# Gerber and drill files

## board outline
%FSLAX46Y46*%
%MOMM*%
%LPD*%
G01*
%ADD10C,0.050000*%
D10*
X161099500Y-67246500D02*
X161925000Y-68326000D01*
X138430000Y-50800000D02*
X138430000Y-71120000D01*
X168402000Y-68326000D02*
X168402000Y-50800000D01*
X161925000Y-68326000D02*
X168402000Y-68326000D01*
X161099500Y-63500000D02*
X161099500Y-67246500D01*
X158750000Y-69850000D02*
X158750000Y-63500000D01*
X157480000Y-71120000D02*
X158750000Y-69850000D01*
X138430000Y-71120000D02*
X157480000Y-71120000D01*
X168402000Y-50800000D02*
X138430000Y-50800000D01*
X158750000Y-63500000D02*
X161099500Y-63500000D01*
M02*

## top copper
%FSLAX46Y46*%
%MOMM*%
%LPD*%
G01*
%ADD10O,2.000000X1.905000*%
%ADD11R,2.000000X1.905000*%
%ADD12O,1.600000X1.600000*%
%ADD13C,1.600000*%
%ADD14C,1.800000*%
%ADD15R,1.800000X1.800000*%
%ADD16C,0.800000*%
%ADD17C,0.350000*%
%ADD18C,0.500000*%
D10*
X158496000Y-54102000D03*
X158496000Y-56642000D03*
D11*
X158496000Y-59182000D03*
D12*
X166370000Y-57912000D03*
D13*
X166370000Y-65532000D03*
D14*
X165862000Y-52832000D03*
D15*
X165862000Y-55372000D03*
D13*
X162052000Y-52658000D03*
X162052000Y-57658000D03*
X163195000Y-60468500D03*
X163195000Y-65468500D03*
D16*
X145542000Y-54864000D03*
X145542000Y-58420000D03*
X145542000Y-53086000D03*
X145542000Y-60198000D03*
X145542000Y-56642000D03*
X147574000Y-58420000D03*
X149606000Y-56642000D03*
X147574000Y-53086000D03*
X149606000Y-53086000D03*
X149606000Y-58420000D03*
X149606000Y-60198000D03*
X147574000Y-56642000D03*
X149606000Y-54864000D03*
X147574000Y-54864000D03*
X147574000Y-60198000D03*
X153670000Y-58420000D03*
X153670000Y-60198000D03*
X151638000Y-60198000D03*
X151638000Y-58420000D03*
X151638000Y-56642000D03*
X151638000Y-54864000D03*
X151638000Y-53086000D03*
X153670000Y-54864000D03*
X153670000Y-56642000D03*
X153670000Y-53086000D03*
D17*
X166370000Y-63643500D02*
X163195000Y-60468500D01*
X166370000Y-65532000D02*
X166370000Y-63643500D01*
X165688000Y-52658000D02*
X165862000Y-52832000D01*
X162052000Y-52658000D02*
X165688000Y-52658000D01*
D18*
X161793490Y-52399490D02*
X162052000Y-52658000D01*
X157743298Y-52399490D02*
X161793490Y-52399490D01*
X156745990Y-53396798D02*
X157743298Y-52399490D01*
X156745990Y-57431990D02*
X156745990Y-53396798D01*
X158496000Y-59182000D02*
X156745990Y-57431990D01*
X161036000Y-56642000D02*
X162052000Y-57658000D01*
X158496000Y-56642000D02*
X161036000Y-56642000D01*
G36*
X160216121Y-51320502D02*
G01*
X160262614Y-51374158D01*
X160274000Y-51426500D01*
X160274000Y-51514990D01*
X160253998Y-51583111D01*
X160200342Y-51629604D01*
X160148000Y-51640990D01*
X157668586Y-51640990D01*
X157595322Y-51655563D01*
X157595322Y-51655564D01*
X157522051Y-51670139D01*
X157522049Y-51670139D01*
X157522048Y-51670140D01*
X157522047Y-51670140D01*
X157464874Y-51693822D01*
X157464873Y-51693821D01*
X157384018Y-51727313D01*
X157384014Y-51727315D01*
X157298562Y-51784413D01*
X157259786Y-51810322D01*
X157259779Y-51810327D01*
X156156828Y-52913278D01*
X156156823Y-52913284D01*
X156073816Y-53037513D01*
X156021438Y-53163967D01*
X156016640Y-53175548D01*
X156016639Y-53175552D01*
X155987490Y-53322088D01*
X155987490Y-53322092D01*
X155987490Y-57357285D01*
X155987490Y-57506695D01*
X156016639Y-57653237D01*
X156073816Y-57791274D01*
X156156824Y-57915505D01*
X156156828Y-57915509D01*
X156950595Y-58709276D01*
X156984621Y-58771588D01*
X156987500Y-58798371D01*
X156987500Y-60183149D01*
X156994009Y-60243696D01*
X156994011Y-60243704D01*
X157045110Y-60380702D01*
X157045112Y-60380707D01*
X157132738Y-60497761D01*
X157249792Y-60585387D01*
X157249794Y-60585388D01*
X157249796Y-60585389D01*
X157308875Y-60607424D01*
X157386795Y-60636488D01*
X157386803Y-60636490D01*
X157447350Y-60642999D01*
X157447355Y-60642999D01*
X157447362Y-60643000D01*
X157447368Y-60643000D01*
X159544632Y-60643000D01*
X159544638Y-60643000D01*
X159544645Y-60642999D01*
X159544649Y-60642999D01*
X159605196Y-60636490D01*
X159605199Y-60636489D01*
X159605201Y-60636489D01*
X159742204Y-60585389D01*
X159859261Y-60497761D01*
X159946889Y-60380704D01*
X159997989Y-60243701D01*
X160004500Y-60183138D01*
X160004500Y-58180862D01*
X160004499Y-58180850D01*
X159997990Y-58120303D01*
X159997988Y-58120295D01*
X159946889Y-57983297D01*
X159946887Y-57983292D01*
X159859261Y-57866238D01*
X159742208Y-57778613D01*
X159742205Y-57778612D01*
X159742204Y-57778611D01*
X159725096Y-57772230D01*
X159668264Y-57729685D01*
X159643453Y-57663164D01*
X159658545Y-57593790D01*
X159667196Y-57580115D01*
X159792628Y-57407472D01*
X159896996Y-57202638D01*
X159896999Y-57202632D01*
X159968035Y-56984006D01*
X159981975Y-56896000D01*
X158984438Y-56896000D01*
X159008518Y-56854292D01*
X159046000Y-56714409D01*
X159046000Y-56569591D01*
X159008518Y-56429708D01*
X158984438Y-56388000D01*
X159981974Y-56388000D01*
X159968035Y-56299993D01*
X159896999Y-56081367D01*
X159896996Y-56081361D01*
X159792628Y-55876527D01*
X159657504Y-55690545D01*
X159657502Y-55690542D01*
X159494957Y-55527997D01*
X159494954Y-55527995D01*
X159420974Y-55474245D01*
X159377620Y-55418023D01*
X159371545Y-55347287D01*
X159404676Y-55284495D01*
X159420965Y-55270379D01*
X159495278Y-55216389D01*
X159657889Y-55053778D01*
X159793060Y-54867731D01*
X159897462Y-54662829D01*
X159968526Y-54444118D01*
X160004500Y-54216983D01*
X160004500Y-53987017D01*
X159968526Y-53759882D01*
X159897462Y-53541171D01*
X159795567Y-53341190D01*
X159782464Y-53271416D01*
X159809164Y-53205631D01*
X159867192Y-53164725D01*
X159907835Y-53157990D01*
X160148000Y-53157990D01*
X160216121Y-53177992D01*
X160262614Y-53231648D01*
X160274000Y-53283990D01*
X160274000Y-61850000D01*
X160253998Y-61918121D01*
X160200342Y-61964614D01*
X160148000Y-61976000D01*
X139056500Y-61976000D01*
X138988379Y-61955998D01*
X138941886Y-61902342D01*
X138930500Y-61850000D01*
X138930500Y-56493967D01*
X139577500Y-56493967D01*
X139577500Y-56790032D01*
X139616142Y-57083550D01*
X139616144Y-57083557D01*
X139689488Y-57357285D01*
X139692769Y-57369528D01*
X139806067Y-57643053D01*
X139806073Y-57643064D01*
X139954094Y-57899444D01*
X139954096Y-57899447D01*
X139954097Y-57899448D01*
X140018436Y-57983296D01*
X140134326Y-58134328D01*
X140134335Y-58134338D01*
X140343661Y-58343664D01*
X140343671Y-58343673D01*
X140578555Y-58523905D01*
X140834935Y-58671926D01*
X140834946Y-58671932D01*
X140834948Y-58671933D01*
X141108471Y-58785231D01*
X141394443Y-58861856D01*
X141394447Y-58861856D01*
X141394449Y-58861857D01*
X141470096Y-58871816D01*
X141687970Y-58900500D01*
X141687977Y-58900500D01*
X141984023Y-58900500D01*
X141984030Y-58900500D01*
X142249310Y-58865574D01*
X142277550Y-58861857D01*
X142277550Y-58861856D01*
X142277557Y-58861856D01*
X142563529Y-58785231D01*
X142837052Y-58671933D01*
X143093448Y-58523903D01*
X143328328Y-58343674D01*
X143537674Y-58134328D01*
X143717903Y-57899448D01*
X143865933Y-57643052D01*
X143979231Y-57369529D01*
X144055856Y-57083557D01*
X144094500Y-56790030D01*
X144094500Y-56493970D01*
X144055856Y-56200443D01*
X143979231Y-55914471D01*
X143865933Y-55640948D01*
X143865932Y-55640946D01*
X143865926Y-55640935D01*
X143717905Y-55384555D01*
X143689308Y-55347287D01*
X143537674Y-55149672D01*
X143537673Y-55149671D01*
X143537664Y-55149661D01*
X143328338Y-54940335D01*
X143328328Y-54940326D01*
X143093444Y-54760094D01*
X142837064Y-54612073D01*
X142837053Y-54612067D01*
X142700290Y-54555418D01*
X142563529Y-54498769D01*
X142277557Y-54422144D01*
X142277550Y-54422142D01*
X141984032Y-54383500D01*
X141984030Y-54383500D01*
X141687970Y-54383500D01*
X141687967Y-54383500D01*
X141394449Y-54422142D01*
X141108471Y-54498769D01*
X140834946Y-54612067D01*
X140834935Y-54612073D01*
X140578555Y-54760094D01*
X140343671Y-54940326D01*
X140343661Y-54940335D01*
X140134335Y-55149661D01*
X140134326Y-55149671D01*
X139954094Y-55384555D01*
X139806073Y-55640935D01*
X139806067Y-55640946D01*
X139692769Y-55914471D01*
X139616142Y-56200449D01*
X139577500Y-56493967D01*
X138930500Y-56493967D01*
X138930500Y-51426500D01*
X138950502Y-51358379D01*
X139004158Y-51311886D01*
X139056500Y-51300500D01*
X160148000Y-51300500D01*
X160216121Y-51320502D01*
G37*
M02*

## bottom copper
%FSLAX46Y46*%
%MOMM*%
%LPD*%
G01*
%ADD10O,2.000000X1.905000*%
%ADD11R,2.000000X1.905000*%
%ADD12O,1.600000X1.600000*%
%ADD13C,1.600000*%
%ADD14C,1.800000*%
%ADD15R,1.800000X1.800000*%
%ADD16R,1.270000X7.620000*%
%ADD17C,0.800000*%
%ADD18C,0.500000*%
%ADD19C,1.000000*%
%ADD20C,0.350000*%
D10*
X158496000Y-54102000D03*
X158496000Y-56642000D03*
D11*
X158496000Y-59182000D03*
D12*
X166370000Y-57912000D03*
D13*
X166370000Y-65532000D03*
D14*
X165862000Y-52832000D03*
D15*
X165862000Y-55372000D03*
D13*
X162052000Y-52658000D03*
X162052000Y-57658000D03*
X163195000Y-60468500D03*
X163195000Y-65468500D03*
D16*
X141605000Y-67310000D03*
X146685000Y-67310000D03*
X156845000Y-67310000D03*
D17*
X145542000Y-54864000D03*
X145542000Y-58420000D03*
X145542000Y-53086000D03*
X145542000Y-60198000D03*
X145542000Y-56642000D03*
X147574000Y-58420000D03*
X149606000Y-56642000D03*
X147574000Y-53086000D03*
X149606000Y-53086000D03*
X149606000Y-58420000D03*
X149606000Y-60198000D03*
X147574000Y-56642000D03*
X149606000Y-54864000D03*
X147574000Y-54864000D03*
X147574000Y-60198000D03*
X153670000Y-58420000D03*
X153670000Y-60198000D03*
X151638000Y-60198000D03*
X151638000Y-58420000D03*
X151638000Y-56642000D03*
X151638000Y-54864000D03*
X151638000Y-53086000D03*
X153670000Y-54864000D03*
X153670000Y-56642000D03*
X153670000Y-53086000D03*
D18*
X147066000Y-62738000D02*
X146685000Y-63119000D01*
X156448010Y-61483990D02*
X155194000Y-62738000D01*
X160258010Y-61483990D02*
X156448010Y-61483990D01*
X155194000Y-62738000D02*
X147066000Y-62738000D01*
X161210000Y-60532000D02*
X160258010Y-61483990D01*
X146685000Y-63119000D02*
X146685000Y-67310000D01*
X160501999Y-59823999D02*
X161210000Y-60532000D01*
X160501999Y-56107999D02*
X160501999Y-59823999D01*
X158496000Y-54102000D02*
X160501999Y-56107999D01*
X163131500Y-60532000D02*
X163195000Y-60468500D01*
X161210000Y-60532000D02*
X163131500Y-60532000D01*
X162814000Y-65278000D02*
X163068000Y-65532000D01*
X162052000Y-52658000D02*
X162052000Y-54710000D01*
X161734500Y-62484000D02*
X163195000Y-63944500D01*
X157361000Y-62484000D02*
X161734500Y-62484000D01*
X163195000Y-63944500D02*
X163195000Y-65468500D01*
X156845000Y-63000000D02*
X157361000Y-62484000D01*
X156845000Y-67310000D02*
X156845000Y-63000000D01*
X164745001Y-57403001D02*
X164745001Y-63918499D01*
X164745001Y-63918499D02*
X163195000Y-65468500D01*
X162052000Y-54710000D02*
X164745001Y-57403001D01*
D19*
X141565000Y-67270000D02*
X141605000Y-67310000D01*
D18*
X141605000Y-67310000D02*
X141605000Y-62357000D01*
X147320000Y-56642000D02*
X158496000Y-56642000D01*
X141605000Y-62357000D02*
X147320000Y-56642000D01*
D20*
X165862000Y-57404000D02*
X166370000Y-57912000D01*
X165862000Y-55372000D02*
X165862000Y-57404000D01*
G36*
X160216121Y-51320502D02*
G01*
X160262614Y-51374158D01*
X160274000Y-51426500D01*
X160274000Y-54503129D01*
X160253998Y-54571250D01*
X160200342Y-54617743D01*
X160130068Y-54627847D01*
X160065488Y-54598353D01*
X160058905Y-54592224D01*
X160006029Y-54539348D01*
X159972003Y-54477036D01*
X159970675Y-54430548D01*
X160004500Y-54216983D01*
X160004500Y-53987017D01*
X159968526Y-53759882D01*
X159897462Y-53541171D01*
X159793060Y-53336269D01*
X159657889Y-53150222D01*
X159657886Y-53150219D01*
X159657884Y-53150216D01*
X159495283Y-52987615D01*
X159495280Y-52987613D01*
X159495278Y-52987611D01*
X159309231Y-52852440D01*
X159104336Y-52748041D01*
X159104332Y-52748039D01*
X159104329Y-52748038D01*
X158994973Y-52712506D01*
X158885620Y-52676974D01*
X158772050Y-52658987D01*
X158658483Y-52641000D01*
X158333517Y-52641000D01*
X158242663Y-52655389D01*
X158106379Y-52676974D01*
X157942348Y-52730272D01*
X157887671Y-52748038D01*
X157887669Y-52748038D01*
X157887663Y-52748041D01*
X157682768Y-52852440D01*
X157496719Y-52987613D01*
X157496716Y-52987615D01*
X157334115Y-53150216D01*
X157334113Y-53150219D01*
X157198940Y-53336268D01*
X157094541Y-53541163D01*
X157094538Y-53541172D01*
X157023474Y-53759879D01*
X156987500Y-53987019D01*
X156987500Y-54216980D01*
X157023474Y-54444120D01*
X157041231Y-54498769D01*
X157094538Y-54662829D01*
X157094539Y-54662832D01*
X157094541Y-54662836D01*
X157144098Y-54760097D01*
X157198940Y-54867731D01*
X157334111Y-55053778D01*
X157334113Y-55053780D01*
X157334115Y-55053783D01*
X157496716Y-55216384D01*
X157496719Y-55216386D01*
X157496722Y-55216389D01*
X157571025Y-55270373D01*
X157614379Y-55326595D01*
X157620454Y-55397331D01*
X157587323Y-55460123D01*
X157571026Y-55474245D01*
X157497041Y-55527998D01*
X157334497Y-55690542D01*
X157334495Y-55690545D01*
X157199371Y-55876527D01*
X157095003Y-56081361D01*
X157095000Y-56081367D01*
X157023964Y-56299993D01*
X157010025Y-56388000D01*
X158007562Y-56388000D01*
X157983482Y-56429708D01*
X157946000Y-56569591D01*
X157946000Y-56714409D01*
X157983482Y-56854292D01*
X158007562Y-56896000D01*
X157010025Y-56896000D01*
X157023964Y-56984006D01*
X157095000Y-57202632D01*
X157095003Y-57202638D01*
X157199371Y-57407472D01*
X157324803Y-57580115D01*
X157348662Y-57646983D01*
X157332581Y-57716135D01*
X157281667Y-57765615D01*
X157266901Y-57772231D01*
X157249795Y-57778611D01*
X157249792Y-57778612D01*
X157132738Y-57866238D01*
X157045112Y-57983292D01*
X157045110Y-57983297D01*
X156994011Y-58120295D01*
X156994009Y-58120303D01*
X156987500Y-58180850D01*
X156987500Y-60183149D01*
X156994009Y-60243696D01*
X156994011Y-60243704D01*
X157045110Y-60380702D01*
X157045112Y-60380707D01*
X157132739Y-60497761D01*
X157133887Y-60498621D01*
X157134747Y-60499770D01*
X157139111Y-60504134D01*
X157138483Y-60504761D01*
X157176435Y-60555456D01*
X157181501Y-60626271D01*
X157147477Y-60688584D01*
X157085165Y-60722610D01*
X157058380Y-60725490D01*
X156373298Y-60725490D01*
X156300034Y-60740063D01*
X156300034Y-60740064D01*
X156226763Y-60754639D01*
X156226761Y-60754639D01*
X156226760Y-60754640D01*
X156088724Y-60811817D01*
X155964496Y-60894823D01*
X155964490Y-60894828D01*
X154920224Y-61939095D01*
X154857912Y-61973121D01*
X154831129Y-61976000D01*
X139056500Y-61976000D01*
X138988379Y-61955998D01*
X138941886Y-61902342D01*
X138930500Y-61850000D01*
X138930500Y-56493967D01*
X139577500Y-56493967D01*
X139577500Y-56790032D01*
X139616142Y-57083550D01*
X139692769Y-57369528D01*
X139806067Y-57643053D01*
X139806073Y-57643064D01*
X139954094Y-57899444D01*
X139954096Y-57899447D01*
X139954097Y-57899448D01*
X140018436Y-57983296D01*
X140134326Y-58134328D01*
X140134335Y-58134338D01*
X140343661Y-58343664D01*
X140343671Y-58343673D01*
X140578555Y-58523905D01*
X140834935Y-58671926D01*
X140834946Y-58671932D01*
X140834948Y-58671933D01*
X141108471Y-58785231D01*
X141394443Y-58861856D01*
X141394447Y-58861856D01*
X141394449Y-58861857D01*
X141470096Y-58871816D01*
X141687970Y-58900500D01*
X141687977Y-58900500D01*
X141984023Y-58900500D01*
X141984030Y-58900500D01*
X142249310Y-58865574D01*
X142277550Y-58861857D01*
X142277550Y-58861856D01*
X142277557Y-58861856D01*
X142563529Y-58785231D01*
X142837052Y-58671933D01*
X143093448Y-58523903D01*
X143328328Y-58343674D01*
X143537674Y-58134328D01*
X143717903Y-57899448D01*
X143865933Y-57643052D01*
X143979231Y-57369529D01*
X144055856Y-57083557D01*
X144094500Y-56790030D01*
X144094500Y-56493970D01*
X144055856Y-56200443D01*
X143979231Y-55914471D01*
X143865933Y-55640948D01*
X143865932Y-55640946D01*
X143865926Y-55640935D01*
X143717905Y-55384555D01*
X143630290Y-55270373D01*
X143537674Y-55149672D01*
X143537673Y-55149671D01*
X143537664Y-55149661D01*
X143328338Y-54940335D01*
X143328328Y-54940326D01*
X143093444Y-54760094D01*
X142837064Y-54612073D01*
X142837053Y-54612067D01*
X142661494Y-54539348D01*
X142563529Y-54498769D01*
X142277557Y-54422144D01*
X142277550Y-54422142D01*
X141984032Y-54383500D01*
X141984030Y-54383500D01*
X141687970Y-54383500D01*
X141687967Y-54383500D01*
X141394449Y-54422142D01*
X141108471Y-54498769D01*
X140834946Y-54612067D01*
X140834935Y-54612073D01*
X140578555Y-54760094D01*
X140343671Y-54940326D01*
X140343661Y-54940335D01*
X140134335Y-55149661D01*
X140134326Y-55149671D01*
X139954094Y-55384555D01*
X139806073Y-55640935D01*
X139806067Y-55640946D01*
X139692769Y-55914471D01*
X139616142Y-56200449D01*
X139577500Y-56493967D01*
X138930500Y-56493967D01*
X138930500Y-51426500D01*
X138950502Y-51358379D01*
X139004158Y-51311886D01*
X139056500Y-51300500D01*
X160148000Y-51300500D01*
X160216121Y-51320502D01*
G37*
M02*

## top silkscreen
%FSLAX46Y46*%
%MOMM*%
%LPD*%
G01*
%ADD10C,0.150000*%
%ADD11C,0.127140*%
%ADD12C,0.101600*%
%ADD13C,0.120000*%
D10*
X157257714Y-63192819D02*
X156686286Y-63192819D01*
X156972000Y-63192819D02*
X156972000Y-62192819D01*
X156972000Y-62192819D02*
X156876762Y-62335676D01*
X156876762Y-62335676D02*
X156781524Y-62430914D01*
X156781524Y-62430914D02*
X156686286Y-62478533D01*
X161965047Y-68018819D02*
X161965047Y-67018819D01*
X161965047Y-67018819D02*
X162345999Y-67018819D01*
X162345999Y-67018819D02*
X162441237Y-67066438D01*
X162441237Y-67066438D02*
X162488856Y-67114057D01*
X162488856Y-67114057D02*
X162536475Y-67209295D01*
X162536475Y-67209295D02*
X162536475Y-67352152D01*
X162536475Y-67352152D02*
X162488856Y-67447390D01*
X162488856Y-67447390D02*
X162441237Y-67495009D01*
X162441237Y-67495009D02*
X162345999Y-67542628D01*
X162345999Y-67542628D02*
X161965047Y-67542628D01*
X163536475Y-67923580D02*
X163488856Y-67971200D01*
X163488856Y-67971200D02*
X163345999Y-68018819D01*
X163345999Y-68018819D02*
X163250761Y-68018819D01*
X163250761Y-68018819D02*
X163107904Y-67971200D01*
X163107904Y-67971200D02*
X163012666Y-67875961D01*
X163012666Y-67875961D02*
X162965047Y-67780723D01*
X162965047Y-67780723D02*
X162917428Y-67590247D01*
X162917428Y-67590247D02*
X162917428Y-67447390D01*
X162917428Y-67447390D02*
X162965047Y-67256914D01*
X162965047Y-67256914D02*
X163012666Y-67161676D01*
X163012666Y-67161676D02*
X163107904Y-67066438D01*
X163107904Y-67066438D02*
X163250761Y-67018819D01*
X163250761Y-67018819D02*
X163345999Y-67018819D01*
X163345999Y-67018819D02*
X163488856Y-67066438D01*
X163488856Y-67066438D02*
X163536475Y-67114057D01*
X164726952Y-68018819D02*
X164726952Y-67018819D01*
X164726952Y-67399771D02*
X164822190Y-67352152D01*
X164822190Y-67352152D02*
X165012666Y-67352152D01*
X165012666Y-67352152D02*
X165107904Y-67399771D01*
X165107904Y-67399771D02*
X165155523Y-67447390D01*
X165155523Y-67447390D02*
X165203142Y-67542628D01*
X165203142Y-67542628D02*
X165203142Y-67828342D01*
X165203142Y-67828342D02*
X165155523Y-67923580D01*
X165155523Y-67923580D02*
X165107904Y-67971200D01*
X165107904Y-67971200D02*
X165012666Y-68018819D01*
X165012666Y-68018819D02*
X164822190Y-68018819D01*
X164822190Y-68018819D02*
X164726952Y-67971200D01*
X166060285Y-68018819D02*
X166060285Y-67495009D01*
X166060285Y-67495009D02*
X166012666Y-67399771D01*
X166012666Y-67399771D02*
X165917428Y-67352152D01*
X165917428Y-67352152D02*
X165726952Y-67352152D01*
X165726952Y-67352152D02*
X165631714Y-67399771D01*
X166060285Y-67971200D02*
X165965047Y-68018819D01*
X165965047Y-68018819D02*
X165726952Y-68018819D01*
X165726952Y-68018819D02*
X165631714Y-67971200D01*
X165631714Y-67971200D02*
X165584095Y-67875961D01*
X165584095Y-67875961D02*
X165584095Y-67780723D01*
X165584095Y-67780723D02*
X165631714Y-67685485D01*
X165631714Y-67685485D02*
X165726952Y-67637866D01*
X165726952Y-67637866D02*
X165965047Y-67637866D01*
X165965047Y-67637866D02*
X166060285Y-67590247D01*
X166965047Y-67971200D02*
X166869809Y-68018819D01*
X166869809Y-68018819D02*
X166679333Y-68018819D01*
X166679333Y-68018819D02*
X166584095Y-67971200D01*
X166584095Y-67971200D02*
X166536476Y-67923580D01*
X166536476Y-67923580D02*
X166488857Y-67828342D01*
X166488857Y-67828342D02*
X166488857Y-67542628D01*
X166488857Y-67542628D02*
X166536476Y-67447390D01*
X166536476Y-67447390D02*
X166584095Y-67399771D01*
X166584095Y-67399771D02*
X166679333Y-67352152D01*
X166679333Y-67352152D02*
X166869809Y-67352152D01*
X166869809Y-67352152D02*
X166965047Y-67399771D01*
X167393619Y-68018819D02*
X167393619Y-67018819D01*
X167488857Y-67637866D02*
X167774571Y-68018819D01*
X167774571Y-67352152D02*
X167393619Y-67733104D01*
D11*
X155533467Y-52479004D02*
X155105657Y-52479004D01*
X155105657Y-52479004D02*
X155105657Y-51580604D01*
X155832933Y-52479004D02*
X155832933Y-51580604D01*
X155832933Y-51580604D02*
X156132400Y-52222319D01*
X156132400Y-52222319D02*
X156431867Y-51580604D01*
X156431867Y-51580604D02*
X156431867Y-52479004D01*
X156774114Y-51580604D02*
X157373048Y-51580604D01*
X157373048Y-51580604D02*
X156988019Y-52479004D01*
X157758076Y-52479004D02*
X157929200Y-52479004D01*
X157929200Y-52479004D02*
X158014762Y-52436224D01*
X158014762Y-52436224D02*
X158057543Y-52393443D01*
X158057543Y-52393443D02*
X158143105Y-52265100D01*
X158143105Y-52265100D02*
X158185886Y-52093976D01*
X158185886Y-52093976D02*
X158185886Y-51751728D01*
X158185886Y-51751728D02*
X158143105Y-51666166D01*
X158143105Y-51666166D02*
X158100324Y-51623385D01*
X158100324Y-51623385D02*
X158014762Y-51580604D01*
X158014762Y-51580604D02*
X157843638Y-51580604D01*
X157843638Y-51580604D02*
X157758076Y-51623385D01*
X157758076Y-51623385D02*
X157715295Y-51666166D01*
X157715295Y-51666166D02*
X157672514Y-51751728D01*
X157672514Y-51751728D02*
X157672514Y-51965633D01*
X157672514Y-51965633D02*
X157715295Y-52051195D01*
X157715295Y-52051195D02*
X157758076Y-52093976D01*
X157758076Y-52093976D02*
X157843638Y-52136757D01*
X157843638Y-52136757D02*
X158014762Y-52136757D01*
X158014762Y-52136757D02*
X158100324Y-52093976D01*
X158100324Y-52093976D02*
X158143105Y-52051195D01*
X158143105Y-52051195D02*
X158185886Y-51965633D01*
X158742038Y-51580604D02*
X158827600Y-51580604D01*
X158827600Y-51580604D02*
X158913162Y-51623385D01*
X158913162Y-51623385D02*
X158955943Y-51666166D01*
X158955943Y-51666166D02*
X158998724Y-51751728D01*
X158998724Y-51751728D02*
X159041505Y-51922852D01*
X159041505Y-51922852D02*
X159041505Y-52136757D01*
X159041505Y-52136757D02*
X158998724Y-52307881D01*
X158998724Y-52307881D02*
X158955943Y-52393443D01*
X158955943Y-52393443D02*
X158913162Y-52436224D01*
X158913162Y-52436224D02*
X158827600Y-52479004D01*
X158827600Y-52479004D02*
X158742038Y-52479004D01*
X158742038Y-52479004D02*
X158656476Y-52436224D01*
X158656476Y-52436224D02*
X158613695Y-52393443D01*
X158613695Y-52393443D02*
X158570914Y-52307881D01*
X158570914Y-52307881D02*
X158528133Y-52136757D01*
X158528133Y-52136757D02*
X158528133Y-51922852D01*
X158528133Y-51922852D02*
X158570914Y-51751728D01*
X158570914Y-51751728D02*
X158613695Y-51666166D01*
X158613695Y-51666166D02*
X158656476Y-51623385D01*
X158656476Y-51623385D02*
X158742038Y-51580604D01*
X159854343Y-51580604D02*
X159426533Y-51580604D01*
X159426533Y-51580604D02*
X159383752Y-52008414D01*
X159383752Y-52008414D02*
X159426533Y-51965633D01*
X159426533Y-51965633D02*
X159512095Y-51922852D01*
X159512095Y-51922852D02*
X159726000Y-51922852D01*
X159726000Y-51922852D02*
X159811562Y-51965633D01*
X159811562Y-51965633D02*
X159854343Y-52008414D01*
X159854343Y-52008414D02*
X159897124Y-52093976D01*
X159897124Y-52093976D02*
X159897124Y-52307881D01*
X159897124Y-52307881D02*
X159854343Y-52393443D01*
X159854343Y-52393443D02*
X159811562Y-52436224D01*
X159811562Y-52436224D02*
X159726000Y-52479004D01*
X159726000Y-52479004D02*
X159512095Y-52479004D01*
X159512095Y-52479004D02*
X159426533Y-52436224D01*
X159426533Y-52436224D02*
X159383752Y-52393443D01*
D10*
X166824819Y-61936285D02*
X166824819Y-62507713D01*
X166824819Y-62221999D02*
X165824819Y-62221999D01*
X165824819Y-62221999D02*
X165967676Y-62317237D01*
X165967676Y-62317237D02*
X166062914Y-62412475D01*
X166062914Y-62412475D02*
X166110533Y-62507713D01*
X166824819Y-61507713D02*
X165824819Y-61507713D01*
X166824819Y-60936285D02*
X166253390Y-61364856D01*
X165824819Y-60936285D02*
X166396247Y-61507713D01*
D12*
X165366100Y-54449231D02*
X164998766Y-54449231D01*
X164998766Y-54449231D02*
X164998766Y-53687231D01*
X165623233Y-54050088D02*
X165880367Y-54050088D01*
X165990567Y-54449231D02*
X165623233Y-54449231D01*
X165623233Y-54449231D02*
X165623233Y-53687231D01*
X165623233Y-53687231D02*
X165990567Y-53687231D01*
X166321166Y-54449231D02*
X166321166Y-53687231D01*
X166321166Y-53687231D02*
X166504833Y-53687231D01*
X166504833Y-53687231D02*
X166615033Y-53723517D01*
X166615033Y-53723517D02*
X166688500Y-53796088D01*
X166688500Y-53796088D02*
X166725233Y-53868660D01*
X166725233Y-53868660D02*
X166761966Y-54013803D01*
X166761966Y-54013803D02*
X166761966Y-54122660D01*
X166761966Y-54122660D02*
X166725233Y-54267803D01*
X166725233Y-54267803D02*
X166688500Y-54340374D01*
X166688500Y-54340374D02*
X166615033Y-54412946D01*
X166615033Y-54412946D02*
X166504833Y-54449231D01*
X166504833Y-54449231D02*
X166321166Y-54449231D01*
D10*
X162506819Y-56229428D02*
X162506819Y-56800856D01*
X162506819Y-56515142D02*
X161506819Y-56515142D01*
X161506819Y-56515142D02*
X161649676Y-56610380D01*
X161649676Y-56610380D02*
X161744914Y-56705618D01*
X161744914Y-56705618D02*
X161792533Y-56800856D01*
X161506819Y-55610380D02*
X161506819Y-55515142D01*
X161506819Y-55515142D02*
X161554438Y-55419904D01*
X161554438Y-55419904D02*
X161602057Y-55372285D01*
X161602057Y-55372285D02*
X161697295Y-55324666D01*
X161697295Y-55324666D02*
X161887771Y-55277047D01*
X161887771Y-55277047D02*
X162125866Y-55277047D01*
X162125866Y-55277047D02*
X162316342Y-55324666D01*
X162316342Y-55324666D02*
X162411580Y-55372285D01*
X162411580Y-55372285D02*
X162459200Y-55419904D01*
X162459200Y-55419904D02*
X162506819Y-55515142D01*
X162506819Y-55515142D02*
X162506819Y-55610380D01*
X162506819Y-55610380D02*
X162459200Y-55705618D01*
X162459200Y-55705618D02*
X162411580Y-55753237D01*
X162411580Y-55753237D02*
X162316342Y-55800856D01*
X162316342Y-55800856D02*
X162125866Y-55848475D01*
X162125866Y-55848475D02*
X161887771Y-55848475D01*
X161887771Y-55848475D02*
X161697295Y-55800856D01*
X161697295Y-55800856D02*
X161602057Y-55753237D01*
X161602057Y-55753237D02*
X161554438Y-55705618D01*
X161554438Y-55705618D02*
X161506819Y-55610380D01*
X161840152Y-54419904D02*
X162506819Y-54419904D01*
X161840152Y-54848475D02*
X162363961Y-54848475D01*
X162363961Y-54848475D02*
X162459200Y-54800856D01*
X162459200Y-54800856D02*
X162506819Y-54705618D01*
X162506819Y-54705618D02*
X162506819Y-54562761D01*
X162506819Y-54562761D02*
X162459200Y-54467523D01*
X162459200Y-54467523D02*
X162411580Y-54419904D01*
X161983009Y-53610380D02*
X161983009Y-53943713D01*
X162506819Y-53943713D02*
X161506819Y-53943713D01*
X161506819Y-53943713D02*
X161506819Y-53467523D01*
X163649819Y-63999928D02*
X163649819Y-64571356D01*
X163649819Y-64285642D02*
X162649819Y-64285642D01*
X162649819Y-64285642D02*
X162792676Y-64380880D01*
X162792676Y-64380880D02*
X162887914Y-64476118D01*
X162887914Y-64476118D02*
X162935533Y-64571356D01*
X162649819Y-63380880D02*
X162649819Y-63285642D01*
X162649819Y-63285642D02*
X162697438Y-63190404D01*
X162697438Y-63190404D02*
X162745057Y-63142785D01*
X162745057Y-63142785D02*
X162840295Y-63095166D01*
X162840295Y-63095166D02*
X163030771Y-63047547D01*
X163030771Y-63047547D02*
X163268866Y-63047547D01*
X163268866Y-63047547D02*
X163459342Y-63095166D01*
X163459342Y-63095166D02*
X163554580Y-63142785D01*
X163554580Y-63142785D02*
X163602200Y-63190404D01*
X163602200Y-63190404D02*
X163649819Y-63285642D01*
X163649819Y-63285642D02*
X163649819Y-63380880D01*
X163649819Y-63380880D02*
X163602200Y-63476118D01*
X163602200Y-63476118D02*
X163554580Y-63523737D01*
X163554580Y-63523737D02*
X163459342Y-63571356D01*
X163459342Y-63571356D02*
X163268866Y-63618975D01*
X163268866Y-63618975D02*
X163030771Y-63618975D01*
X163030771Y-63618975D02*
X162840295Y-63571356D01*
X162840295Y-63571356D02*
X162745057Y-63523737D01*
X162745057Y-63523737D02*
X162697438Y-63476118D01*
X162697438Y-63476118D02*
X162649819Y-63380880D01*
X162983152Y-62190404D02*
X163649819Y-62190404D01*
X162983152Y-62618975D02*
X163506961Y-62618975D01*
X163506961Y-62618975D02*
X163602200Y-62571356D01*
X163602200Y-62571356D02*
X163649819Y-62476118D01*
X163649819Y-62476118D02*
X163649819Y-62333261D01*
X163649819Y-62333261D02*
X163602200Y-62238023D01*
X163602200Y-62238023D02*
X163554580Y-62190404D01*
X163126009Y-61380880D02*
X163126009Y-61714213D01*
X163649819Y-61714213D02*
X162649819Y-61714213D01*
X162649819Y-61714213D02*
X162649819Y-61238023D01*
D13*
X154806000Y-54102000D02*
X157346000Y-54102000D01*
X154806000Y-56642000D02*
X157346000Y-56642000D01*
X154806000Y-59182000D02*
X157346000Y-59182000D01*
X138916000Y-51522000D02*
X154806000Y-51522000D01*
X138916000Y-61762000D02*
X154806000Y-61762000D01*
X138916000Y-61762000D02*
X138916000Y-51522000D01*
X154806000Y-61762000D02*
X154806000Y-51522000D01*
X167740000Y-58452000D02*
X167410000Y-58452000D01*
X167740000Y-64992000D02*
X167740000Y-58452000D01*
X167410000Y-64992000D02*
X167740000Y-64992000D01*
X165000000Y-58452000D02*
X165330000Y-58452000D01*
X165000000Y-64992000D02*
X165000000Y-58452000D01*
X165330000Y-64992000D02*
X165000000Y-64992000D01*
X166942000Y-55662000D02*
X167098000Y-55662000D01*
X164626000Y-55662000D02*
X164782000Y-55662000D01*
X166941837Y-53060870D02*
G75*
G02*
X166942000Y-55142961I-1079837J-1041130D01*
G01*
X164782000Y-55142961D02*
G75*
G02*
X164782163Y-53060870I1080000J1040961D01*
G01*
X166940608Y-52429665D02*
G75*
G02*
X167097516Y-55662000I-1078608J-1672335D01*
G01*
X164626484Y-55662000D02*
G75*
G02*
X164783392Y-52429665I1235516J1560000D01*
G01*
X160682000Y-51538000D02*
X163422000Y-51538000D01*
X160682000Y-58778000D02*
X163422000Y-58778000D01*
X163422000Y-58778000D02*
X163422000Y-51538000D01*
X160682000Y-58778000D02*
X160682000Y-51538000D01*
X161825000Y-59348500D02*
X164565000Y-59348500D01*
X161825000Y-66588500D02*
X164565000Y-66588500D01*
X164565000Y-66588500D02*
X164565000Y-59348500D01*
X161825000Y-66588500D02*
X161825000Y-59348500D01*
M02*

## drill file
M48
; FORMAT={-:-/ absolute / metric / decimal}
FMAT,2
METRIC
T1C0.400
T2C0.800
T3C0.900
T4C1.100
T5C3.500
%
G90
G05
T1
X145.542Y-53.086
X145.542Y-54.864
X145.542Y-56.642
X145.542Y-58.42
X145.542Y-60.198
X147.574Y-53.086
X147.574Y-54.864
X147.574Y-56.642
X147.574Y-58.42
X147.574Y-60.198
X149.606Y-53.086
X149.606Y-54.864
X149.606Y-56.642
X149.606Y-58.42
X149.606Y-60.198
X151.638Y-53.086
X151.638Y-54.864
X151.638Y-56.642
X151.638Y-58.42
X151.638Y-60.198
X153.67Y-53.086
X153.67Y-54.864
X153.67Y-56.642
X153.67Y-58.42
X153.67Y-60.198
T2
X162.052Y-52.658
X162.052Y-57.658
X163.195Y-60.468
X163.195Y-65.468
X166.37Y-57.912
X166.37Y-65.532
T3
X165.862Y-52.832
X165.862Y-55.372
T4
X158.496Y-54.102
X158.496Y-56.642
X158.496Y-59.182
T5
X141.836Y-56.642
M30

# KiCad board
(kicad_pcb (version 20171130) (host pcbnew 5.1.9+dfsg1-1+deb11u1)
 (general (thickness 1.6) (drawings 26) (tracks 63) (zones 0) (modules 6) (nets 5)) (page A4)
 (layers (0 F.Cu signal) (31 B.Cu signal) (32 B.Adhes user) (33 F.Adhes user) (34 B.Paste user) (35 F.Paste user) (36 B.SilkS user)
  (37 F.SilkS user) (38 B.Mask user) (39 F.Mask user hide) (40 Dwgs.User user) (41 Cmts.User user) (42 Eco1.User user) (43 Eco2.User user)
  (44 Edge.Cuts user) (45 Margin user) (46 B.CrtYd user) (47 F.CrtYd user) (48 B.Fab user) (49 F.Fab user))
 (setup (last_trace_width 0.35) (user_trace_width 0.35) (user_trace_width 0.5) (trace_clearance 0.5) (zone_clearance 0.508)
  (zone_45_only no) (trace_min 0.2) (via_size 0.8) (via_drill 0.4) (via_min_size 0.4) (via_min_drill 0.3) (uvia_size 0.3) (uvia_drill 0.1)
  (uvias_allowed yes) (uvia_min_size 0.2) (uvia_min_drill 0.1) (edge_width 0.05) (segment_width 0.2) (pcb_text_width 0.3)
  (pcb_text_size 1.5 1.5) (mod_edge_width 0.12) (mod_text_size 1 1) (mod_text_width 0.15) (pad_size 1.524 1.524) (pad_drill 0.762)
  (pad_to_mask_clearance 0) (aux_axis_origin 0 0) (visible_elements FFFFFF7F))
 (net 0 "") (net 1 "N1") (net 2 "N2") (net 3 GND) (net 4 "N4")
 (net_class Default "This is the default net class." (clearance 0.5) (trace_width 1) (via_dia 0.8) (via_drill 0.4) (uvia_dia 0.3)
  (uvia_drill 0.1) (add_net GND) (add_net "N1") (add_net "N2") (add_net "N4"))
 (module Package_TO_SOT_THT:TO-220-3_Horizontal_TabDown (layer F.Cu) (at 158.496 59.182 90)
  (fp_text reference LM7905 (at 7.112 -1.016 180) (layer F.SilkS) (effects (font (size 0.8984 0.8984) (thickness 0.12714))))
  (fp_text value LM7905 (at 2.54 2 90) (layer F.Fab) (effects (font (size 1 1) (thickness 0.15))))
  (fp_line (start 5.08 -3.69) (end 5.08 -1.15) (layer F.SilkS) (width 0.12))
  (fp_line (start 2.54 -3.69) (end 2.54 -1.15) (layer F.SilkS) (width 0.12))
  (fp_line (start 0 -3.69) (end 0 -1.15) (layer F.SilkS) (width 0.12))
  (fp_line (start 7.66 -19.58) (end 7.66 -3.69) (layer F.SilkS) (width 0.12))
  (fp_line (start -2.58 -19.58) (end -2.58 -3.69) (layer F.SilkS) (width 0.12))
  (fp_line (start -2.58 -19.58) (end 7.66 -19.58) (layer F.SilkS) (width 0.12))
  (fp_line (start -2.58 -3.69) (end 7.66 -3.69) (layer F.SilkS) (width 0.12))
  (pad 3 thru_hole oval (at 5.08 0 90) (size 1.905 2) (drill 1.1) (layers *.Cu *.Mask) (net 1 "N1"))
  (pad 2 thru_hole oval (at 2.54 0 90) (size 1.905 2) (drill 1.1) (layers *.Cu *.Mask) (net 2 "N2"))
  (pad 1 thru_hole rect (at 0 0 90) (size 1.905 2) (drill 1.1) (layers *.Cu *.Mask) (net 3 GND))
  (pad "" np_thru_hole oval (at 2.54 -16.66 90) (size 3.5 3.5) (drill 3.5) (layers *.Cu *.Mask)))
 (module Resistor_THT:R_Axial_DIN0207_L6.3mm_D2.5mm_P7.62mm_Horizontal (layer F.Cu) (at 166.37 65.532 90)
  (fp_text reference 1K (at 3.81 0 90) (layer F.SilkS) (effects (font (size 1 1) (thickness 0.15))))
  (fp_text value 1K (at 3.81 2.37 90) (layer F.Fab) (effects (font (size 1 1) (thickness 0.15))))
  (fp_line (start 7.08 1.37) (end 7.08 1.04) (layer F.SilkS) (width 0.12))
  (fp_line (start 0.54 1.37) (end 7.08 1.37) (layer F.SilkS) (width 0.12))
  (fp_line (start 0.54 1.04) (end 0.54 1.37) (layer F.SilkS) (width 0.12))
  (fp_line (start 7.08 -1.37) (end 7.08 -1.04) (layer F.SilkS) (width 0.12))
  (fp_line (start 0.54 -1.37) (end 7.08 -1.37) (layer F.SilkS) (width 0.12))
  (fp_line (start 0.54 -1.04) (end 0.54 -1.37) (layer F.SilkS) (width 0.12))
  (pad 2 thru_hole oval (at 7.62 0 90) (size 1.6 1.6) (drill 0.8) (layers *.Cu *.Mask) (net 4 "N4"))
  (pad 1 thru_hole circle (at 0 0 90) (size 1.6 1.6) (drill 0.8) (layers *.Cu *.Mask) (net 1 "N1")))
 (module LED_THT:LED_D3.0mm (layer F.Cu) (at 165.862 55.372 90)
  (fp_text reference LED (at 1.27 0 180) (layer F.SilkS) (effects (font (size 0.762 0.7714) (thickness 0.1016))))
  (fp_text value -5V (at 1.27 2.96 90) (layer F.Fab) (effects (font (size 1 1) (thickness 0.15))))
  (fp_line (start -0.29 1.08) (end -0.29 1.236) (layer F.SilkS) (width 0.12))
  (fp_line (start -0.29 -1.236) (end -0.29 -1.08) (layer F.SilkS) (width 0.12))
  (fp_arc (start 1.27 0) (end 0.229039 1.08) (angle -87.9) (layer F.SilkS) (width 0.12))
  (fp_arc (start 1.27 0) (end 0.229039 -1.08) (angle 87.9) (layer F.SilkS) (width 0.12))
  (fp_arc (start 1.27 0) (end -0.29 1.235516) (angle -108.8) (layer F.SilkS) (width 0.12))
  (fp_arc (start 1.27 0) (end -0.29 -1.235516) (angle 108.8) (layer F.SilkS) (width 0.12))
  (pad 2 thru_hole circle (at 2.54 0 90) (size 1.8 1.8) (drill 0.9) (layers *.Cu *.Mask) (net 3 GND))
  (pad 1 thru_hole rect (at 0 0 90) (size 1.8 1.8) (drill 0.9) (layers *.Cu *.Mask) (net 4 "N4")))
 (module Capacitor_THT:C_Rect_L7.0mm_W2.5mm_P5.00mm (layer F.Cu) (at 162.052 57.658 90)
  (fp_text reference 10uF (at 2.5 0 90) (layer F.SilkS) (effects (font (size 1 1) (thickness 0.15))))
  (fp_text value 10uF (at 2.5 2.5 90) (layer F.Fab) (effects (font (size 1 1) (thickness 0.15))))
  (fp_line (start 6.12 -1.37) (end 6.12 1.37) (layer F.SilkS) (width 0.12))
  (fp_line (start -1.12 -1.37) (end -1.12 1.37) (layer F.SilkS) (width 0.12))
  (fp_line (start -1.12 1.37) (end 6.12 1.37) (layer F.SilkS) (width 0.12))
  (fp_line (start -1.12 -1.37) (end 6.12 -1.37) (layer F.SilkS) (width 0.12))
  (pad 2 thru_hole circle (at 5 0 90) (size 1.6 1.6) (drill 0.8) (layers *.Cu *.Mask) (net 3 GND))
  (pad 1 thru_hole circle (at 0 0 90) (size 1.6 1.6) (drill 0.8) (layers *.Cu *.Mask) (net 2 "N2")))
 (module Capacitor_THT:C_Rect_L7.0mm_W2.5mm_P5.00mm (layer F.Cu) (at 163.195 65.4685 90)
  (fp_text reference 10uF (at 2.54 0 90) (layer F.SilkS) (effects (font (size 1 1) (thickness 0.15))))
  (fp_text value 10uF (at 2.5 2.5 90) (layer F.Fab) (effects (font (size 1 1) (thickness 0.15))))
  (fp_line (start 6.12 -1.37) (end 6.12 1.37) (layer F.SilkS) (width 0.12))
  (fp_line (start -1.12 -1.37) (end -1.12 1.37) (layer F.SilkS) (width 0.12))
  (fp_line (start -1.12 1.37) (end 6.12 1.37) (layer F.SilkS) (width 0.12))
  (fp_line (start -1.12 -1.37) (end 6.12 -1.37) (layer F.SilkS) (width 0.12))
  (pad 2 thru_hole circle (at 5 0 90) (size 1.6 1.6) (drill 0.8) (layers *.Cu *.Mask) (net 1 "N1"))
  (pad 1 thru_hole circle (at 0 0 90) (size 1.6 1.6) (drill 0.8) (layers *.Cu *.Mask) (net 3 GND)))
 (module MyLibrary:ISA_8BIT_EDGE (layer F.Cu) (at 156.845 63.5)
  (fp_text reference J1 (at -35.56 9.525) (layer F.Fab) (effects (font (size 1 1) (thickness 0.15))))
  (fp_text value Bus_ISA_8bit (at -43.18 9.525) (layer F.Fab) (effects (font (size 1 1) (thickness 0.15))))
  (pad 7 connect rect (at -15.24 3.81) (size 1.27 7.62) (layers B.Cu B.Mask) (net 2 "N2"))
  (pad 5 connect rect (at -10.16 3.81) (size 1.27 7.62) (layers B.Cu B.Mask) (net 1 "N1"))
  (pad 1 connect rect (at 0 3.81) (size 1.27 7.62) (layers B.Cu B.Mask) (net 3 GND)))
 (gr_line (start 161.0995 67.2465) (end 161.925 68.326) (layer Edge.Cuts) (width 0.05))
 (gr_line (start 138.43 50.8) (end 138.43 71.12) (layer Edge.Cuts) (width 0.05))
 (gr_line (start 168.402 68.326) (end 168.402 50.8) (layer Edge.Cuts) (width 0.05))
 (gr_line (start 161.925 68.326) (end 168.402 68.326) (layer Edge.Cuts) (width 0.05))
 (gr_line (start 161.0995 63.5) (end 161.0995 67.2465) (layer Edge.Cuts) (width 0.05))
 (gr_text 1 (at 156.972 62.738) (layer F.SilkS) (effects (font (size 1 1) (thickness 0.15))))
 (gr_line (start 158.75 69.85) (end 158.75 63.5) (layer Edge.Cuts) (width 0.05))
 (gr_line (start 157.48 71.12) (end 158.75 69.85) (layer Edge.Cuts) (width 0.05))
 (gr_line (start 138.43 71.12) (end 157.48 71.12) (layer Edge.Cuts) (width 0.05))
 (gr_line (start 168.402 50.8) (end 138.43 50.8) (layer Edge.Cuts) (width 0.05))
 (gr_line (start 158.75 63.5) (end 161.0995 63.5) (layer Edge.Cuts) (width 0.05))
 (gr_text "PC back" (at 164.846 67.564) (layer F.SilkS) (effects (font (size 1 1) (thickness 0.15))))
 (segment (start 147.066 62.738) (end 146.685 63.119) (width 0.5) (layer B.Cu) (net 1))
 (segment (start 156.44801 61.48399) (end 155.194 62.738) (width 0.5) (layer B.Cu) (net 1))
 (segment (start 160.25801 61.48399) (end 156.44801 61.48399) (width 0.5) (layer B.Cu) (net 1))
 (segment (start 155.194 62.738) (end 147.066 62.738) (width 0.5) (layer B.Cu) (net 1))
 (segment (start 161.21 60.532) (end 160.25801 61.48399) (width 0.5) (layer B.Cu) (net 1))
 (segment (start 146.685 63.119) (end 146.685 67.31) (width 0.5) (layer B.Cu) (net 1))
 (segment (start 160.501999 59.823999) (end 161.21 60.532) (width 0.5) (layer B.Cu) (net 1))
 (segment (start 160.501999 56.107999) (end 160.501999 59.823999) (width 0.5) (layer B.Cu) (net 1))
 (segment (start 158.496 54.102) (end 160.501999 56.107999) (width 0.5) (layer B.Cu) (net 1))
 (segment (start 163.1315 60.532) (end 163.195 60.4685) (width 0.5) (layer B.Cu) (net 1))
 (segment (start 161.21 60.532) (end 163.1315 60.532) (width 0.5) (layer B.Cu) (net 1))
 (segment (start 166.37 63.6435) (end 163.195 60.4685) (width 0.35) (layer F.Cu) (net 1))
 (segment (start 166.37 65.532) (end 166.37 63.6435) (width 0.35) (layer F.Cu) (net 1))
 (segment (start 165.688 52.658) (end 165.862 52.832) (width 0.35) (layer F.Cu) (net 3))
 (segment (start 162.052 52.658) (end 165.688 52.658) (width 0.35) (layer F.Cu) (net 3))
 (segment (start 161.79349 52.39949) (end 162.052 52.658) (width 0.5) (layer F.Cu) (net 3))
 (segment (start 157.743298 52.39949) (end 161.79349 52.39949) (width 0.5) (layer F.Cu) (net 3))
 (segment (start 156.74599 53.396798) (end 157.743298 52.39949) (width 0.5) (layer F.Cu) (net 3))
 (segment (start 156.74599 57.43199) (end 156.74599 53.396798) (width 0.5) (layer F.Cu) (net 3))
 (segment (start 158.496 59.182) (end 156.74599 57.43199) (width 0.5) (layer F.Cu) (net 3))
 (segment (start 162.814 65.278) (end 163.068 65.532) (width 0.5) (layer B.Cu) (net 3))
 (segment (start 162.052 52.658) (end 162.052 54.71) (width 0.5) (layer B.Cu) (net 3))
 (segment (start 161.7345 62.484) (end 163.195 63.9445) (width 0.5) (layer B.Cu) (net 3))
 (segment (start 157.361 62.484) (end 161.7345 62.484) (width 0.5) (layer B.Cu) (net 3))
 (segment (start 163.195 63.9445) (end 163.195 65.4685) (width 0.5) (layer B.Cu) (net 3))
 (segment (start 156.845 63) (end 157.361 62.484) (width 0.5) (layer B.Cu) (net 3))
 (segment (start 156.845 67.31) (end 156.845 63) (width 0.5) (layer B.Cu) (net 3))
 (segment (start 164.745001 57.403001) (end 164.745001 63.918499) (width 0.5) (layer B.Cu) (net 3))
 (segment (start 164.745001 63.918499) (end 163.195 65.4685) (width 0.5) (layer B.Cu) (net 3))
 (segment (start 162.052 54.71) (end 164.745001 57.403001) (width 0.5) (layer B.Cu) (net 3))
 (via (at 145.542 54.864) (size 0.8) (drill 0.4) (layers F.Cu B.Cu) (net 2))
 (via (at 145.542 58.42) (size 0.8) (drill 0.4) (layers F.Cu B.Cu) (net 2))
 (via (at 145.542 53.086) (size 0.8) (drill 0.4) (layers F.Cu B.Cu) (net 2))
 (via (at 145.542 60.198) (size 0.8) (drill 0.4) (layers F.Cu B.Cu) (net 2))
 (via (at 145.542 56.642) (size 0.8) (drill 0.4) (layers F.Cu B.Cu) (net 2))
 (via (at 147.574 58.42) (size 0.8) (drill 0.4) (layers F.Cu B.Cu) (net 2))
 (via (at 149.606 56.642) (size 0.8) (drill 0.4) (layers F.Cu B.Cu) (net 2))
 (via (at 147.574 53.086) (size 0.8) (drill 0.4) (layers F.Cu B.Cu) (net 2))
 (via (at 149.606 53.086) (size 0.8) (drill 0.4) (layers F.Cu B.Cu) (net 2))
 (via (at 149.606 58.42) (size 0.8) (drill 0.4) (layers F.Cu B.Cu) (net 2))
 (via (at 149.606 60.198) (size 0.8) (drill 0.4) (layers F.Cu B.Cu) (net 2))
 (via (at 147.574 56.642) (size 0.8) (drill 0.4) (layers F.Cu B.Cu) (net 2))
 (via (at 149.606 54.864) (size 0.8) (drill 0.4) (layers F.Cu B.Cu) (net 2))
 (via (at 147.574 54.864) (size 0.8) (drill 0.4) (layers F.Cu B.Cu) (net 2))
 (via (at 147.574 60.198) (size 0.8) (drill 0.4) (layers F.Cu B.Cu) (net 2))
 (via (at 153.67 58.42) (size 0.8) (drill 0.4) (layers F.Cu B.Cu) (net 2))
 (via (at 153.67 60.198) (size 0.8) (drill 0.4) (layers F.Cu B.Cu) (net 2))
 (via (at 151.638 60.198) (size 0.8) (drill 0.4) (layers F.Cu B.Cu) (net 2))
 (via (at 151.638 58.42) (size 0.8) (drill 0.4) (layers F.Cu B.Cu) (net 2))
 (via (at 151.638 56.642) (size 0.8) (drill 0.4) (layers F.Cu B.Cu) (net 2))
 (via (at 151.638 54.864) (size 0.8) (drill 0.4) (layers F.Cu B.Cu) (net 2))
 (via (at 151.638 53.086) (size 0.8) (drill 0.4) (layers F.Cu B.Cu) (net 2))
 (via (at 153.67 54.864) (size 0.8) (drill 0.4) (layers F.Cu B.Cu) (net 2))
 (via (at 153.67 56.642) (size 0.8) (drill 0.4) (layers F.Cu B.Cu) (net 2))
 (via (at 153.67 53.086) (size 0.8) (drill 0.4) (layers F.Cu B.Cu) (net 2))
 (segment (start 141.565 67.27) (end 141.605 67.31) (width 1) (layer B.Cu) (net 2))
 (segment (start 141.605 67.31) (end 141.605 62.357) (width 0.5) (layer B.Cu) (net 2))
 (segment (start 147.32 56.642) (end 158.496 56.642) (width 0.5) (layer B.Cu) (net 2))
 (segment (start 141.605 62.357) (end 147.32 56.642) (width 0.5) (layer B.Cu) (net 2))
 (segment (start 161.036 56.642) (end 162.052 57.658) (width 0.5) (layer F.Cu) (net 2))
 (segment (start 158.496 56.642) (end 161.036 56.642) (width 0.5) (layer F.Cu) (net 2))
 (segment (start 165.862 57.404) (end 166.37 57.912) (width 0.35) (layer B.Cu) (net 4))
 (segment (start 165.862 55.372) (end 165.862 57.404) (width 0.35) (layer B.Cu) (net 4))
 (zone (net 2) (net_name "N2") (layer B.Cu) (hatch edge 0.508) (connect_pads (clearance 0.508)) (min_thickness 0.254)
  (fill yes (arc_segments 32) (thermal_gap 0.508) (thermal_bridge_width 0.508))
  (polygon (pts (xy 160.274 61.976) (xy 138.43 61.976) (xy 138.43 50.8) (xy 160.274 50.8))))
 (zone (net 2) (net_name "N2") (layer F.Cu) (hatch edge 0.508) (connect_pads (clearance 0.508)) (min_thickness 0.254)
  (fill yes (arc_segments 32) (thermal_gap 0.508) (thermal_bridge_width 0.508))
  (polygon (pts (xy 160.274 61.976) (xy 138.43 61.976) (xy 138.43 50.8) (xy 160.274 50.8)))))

